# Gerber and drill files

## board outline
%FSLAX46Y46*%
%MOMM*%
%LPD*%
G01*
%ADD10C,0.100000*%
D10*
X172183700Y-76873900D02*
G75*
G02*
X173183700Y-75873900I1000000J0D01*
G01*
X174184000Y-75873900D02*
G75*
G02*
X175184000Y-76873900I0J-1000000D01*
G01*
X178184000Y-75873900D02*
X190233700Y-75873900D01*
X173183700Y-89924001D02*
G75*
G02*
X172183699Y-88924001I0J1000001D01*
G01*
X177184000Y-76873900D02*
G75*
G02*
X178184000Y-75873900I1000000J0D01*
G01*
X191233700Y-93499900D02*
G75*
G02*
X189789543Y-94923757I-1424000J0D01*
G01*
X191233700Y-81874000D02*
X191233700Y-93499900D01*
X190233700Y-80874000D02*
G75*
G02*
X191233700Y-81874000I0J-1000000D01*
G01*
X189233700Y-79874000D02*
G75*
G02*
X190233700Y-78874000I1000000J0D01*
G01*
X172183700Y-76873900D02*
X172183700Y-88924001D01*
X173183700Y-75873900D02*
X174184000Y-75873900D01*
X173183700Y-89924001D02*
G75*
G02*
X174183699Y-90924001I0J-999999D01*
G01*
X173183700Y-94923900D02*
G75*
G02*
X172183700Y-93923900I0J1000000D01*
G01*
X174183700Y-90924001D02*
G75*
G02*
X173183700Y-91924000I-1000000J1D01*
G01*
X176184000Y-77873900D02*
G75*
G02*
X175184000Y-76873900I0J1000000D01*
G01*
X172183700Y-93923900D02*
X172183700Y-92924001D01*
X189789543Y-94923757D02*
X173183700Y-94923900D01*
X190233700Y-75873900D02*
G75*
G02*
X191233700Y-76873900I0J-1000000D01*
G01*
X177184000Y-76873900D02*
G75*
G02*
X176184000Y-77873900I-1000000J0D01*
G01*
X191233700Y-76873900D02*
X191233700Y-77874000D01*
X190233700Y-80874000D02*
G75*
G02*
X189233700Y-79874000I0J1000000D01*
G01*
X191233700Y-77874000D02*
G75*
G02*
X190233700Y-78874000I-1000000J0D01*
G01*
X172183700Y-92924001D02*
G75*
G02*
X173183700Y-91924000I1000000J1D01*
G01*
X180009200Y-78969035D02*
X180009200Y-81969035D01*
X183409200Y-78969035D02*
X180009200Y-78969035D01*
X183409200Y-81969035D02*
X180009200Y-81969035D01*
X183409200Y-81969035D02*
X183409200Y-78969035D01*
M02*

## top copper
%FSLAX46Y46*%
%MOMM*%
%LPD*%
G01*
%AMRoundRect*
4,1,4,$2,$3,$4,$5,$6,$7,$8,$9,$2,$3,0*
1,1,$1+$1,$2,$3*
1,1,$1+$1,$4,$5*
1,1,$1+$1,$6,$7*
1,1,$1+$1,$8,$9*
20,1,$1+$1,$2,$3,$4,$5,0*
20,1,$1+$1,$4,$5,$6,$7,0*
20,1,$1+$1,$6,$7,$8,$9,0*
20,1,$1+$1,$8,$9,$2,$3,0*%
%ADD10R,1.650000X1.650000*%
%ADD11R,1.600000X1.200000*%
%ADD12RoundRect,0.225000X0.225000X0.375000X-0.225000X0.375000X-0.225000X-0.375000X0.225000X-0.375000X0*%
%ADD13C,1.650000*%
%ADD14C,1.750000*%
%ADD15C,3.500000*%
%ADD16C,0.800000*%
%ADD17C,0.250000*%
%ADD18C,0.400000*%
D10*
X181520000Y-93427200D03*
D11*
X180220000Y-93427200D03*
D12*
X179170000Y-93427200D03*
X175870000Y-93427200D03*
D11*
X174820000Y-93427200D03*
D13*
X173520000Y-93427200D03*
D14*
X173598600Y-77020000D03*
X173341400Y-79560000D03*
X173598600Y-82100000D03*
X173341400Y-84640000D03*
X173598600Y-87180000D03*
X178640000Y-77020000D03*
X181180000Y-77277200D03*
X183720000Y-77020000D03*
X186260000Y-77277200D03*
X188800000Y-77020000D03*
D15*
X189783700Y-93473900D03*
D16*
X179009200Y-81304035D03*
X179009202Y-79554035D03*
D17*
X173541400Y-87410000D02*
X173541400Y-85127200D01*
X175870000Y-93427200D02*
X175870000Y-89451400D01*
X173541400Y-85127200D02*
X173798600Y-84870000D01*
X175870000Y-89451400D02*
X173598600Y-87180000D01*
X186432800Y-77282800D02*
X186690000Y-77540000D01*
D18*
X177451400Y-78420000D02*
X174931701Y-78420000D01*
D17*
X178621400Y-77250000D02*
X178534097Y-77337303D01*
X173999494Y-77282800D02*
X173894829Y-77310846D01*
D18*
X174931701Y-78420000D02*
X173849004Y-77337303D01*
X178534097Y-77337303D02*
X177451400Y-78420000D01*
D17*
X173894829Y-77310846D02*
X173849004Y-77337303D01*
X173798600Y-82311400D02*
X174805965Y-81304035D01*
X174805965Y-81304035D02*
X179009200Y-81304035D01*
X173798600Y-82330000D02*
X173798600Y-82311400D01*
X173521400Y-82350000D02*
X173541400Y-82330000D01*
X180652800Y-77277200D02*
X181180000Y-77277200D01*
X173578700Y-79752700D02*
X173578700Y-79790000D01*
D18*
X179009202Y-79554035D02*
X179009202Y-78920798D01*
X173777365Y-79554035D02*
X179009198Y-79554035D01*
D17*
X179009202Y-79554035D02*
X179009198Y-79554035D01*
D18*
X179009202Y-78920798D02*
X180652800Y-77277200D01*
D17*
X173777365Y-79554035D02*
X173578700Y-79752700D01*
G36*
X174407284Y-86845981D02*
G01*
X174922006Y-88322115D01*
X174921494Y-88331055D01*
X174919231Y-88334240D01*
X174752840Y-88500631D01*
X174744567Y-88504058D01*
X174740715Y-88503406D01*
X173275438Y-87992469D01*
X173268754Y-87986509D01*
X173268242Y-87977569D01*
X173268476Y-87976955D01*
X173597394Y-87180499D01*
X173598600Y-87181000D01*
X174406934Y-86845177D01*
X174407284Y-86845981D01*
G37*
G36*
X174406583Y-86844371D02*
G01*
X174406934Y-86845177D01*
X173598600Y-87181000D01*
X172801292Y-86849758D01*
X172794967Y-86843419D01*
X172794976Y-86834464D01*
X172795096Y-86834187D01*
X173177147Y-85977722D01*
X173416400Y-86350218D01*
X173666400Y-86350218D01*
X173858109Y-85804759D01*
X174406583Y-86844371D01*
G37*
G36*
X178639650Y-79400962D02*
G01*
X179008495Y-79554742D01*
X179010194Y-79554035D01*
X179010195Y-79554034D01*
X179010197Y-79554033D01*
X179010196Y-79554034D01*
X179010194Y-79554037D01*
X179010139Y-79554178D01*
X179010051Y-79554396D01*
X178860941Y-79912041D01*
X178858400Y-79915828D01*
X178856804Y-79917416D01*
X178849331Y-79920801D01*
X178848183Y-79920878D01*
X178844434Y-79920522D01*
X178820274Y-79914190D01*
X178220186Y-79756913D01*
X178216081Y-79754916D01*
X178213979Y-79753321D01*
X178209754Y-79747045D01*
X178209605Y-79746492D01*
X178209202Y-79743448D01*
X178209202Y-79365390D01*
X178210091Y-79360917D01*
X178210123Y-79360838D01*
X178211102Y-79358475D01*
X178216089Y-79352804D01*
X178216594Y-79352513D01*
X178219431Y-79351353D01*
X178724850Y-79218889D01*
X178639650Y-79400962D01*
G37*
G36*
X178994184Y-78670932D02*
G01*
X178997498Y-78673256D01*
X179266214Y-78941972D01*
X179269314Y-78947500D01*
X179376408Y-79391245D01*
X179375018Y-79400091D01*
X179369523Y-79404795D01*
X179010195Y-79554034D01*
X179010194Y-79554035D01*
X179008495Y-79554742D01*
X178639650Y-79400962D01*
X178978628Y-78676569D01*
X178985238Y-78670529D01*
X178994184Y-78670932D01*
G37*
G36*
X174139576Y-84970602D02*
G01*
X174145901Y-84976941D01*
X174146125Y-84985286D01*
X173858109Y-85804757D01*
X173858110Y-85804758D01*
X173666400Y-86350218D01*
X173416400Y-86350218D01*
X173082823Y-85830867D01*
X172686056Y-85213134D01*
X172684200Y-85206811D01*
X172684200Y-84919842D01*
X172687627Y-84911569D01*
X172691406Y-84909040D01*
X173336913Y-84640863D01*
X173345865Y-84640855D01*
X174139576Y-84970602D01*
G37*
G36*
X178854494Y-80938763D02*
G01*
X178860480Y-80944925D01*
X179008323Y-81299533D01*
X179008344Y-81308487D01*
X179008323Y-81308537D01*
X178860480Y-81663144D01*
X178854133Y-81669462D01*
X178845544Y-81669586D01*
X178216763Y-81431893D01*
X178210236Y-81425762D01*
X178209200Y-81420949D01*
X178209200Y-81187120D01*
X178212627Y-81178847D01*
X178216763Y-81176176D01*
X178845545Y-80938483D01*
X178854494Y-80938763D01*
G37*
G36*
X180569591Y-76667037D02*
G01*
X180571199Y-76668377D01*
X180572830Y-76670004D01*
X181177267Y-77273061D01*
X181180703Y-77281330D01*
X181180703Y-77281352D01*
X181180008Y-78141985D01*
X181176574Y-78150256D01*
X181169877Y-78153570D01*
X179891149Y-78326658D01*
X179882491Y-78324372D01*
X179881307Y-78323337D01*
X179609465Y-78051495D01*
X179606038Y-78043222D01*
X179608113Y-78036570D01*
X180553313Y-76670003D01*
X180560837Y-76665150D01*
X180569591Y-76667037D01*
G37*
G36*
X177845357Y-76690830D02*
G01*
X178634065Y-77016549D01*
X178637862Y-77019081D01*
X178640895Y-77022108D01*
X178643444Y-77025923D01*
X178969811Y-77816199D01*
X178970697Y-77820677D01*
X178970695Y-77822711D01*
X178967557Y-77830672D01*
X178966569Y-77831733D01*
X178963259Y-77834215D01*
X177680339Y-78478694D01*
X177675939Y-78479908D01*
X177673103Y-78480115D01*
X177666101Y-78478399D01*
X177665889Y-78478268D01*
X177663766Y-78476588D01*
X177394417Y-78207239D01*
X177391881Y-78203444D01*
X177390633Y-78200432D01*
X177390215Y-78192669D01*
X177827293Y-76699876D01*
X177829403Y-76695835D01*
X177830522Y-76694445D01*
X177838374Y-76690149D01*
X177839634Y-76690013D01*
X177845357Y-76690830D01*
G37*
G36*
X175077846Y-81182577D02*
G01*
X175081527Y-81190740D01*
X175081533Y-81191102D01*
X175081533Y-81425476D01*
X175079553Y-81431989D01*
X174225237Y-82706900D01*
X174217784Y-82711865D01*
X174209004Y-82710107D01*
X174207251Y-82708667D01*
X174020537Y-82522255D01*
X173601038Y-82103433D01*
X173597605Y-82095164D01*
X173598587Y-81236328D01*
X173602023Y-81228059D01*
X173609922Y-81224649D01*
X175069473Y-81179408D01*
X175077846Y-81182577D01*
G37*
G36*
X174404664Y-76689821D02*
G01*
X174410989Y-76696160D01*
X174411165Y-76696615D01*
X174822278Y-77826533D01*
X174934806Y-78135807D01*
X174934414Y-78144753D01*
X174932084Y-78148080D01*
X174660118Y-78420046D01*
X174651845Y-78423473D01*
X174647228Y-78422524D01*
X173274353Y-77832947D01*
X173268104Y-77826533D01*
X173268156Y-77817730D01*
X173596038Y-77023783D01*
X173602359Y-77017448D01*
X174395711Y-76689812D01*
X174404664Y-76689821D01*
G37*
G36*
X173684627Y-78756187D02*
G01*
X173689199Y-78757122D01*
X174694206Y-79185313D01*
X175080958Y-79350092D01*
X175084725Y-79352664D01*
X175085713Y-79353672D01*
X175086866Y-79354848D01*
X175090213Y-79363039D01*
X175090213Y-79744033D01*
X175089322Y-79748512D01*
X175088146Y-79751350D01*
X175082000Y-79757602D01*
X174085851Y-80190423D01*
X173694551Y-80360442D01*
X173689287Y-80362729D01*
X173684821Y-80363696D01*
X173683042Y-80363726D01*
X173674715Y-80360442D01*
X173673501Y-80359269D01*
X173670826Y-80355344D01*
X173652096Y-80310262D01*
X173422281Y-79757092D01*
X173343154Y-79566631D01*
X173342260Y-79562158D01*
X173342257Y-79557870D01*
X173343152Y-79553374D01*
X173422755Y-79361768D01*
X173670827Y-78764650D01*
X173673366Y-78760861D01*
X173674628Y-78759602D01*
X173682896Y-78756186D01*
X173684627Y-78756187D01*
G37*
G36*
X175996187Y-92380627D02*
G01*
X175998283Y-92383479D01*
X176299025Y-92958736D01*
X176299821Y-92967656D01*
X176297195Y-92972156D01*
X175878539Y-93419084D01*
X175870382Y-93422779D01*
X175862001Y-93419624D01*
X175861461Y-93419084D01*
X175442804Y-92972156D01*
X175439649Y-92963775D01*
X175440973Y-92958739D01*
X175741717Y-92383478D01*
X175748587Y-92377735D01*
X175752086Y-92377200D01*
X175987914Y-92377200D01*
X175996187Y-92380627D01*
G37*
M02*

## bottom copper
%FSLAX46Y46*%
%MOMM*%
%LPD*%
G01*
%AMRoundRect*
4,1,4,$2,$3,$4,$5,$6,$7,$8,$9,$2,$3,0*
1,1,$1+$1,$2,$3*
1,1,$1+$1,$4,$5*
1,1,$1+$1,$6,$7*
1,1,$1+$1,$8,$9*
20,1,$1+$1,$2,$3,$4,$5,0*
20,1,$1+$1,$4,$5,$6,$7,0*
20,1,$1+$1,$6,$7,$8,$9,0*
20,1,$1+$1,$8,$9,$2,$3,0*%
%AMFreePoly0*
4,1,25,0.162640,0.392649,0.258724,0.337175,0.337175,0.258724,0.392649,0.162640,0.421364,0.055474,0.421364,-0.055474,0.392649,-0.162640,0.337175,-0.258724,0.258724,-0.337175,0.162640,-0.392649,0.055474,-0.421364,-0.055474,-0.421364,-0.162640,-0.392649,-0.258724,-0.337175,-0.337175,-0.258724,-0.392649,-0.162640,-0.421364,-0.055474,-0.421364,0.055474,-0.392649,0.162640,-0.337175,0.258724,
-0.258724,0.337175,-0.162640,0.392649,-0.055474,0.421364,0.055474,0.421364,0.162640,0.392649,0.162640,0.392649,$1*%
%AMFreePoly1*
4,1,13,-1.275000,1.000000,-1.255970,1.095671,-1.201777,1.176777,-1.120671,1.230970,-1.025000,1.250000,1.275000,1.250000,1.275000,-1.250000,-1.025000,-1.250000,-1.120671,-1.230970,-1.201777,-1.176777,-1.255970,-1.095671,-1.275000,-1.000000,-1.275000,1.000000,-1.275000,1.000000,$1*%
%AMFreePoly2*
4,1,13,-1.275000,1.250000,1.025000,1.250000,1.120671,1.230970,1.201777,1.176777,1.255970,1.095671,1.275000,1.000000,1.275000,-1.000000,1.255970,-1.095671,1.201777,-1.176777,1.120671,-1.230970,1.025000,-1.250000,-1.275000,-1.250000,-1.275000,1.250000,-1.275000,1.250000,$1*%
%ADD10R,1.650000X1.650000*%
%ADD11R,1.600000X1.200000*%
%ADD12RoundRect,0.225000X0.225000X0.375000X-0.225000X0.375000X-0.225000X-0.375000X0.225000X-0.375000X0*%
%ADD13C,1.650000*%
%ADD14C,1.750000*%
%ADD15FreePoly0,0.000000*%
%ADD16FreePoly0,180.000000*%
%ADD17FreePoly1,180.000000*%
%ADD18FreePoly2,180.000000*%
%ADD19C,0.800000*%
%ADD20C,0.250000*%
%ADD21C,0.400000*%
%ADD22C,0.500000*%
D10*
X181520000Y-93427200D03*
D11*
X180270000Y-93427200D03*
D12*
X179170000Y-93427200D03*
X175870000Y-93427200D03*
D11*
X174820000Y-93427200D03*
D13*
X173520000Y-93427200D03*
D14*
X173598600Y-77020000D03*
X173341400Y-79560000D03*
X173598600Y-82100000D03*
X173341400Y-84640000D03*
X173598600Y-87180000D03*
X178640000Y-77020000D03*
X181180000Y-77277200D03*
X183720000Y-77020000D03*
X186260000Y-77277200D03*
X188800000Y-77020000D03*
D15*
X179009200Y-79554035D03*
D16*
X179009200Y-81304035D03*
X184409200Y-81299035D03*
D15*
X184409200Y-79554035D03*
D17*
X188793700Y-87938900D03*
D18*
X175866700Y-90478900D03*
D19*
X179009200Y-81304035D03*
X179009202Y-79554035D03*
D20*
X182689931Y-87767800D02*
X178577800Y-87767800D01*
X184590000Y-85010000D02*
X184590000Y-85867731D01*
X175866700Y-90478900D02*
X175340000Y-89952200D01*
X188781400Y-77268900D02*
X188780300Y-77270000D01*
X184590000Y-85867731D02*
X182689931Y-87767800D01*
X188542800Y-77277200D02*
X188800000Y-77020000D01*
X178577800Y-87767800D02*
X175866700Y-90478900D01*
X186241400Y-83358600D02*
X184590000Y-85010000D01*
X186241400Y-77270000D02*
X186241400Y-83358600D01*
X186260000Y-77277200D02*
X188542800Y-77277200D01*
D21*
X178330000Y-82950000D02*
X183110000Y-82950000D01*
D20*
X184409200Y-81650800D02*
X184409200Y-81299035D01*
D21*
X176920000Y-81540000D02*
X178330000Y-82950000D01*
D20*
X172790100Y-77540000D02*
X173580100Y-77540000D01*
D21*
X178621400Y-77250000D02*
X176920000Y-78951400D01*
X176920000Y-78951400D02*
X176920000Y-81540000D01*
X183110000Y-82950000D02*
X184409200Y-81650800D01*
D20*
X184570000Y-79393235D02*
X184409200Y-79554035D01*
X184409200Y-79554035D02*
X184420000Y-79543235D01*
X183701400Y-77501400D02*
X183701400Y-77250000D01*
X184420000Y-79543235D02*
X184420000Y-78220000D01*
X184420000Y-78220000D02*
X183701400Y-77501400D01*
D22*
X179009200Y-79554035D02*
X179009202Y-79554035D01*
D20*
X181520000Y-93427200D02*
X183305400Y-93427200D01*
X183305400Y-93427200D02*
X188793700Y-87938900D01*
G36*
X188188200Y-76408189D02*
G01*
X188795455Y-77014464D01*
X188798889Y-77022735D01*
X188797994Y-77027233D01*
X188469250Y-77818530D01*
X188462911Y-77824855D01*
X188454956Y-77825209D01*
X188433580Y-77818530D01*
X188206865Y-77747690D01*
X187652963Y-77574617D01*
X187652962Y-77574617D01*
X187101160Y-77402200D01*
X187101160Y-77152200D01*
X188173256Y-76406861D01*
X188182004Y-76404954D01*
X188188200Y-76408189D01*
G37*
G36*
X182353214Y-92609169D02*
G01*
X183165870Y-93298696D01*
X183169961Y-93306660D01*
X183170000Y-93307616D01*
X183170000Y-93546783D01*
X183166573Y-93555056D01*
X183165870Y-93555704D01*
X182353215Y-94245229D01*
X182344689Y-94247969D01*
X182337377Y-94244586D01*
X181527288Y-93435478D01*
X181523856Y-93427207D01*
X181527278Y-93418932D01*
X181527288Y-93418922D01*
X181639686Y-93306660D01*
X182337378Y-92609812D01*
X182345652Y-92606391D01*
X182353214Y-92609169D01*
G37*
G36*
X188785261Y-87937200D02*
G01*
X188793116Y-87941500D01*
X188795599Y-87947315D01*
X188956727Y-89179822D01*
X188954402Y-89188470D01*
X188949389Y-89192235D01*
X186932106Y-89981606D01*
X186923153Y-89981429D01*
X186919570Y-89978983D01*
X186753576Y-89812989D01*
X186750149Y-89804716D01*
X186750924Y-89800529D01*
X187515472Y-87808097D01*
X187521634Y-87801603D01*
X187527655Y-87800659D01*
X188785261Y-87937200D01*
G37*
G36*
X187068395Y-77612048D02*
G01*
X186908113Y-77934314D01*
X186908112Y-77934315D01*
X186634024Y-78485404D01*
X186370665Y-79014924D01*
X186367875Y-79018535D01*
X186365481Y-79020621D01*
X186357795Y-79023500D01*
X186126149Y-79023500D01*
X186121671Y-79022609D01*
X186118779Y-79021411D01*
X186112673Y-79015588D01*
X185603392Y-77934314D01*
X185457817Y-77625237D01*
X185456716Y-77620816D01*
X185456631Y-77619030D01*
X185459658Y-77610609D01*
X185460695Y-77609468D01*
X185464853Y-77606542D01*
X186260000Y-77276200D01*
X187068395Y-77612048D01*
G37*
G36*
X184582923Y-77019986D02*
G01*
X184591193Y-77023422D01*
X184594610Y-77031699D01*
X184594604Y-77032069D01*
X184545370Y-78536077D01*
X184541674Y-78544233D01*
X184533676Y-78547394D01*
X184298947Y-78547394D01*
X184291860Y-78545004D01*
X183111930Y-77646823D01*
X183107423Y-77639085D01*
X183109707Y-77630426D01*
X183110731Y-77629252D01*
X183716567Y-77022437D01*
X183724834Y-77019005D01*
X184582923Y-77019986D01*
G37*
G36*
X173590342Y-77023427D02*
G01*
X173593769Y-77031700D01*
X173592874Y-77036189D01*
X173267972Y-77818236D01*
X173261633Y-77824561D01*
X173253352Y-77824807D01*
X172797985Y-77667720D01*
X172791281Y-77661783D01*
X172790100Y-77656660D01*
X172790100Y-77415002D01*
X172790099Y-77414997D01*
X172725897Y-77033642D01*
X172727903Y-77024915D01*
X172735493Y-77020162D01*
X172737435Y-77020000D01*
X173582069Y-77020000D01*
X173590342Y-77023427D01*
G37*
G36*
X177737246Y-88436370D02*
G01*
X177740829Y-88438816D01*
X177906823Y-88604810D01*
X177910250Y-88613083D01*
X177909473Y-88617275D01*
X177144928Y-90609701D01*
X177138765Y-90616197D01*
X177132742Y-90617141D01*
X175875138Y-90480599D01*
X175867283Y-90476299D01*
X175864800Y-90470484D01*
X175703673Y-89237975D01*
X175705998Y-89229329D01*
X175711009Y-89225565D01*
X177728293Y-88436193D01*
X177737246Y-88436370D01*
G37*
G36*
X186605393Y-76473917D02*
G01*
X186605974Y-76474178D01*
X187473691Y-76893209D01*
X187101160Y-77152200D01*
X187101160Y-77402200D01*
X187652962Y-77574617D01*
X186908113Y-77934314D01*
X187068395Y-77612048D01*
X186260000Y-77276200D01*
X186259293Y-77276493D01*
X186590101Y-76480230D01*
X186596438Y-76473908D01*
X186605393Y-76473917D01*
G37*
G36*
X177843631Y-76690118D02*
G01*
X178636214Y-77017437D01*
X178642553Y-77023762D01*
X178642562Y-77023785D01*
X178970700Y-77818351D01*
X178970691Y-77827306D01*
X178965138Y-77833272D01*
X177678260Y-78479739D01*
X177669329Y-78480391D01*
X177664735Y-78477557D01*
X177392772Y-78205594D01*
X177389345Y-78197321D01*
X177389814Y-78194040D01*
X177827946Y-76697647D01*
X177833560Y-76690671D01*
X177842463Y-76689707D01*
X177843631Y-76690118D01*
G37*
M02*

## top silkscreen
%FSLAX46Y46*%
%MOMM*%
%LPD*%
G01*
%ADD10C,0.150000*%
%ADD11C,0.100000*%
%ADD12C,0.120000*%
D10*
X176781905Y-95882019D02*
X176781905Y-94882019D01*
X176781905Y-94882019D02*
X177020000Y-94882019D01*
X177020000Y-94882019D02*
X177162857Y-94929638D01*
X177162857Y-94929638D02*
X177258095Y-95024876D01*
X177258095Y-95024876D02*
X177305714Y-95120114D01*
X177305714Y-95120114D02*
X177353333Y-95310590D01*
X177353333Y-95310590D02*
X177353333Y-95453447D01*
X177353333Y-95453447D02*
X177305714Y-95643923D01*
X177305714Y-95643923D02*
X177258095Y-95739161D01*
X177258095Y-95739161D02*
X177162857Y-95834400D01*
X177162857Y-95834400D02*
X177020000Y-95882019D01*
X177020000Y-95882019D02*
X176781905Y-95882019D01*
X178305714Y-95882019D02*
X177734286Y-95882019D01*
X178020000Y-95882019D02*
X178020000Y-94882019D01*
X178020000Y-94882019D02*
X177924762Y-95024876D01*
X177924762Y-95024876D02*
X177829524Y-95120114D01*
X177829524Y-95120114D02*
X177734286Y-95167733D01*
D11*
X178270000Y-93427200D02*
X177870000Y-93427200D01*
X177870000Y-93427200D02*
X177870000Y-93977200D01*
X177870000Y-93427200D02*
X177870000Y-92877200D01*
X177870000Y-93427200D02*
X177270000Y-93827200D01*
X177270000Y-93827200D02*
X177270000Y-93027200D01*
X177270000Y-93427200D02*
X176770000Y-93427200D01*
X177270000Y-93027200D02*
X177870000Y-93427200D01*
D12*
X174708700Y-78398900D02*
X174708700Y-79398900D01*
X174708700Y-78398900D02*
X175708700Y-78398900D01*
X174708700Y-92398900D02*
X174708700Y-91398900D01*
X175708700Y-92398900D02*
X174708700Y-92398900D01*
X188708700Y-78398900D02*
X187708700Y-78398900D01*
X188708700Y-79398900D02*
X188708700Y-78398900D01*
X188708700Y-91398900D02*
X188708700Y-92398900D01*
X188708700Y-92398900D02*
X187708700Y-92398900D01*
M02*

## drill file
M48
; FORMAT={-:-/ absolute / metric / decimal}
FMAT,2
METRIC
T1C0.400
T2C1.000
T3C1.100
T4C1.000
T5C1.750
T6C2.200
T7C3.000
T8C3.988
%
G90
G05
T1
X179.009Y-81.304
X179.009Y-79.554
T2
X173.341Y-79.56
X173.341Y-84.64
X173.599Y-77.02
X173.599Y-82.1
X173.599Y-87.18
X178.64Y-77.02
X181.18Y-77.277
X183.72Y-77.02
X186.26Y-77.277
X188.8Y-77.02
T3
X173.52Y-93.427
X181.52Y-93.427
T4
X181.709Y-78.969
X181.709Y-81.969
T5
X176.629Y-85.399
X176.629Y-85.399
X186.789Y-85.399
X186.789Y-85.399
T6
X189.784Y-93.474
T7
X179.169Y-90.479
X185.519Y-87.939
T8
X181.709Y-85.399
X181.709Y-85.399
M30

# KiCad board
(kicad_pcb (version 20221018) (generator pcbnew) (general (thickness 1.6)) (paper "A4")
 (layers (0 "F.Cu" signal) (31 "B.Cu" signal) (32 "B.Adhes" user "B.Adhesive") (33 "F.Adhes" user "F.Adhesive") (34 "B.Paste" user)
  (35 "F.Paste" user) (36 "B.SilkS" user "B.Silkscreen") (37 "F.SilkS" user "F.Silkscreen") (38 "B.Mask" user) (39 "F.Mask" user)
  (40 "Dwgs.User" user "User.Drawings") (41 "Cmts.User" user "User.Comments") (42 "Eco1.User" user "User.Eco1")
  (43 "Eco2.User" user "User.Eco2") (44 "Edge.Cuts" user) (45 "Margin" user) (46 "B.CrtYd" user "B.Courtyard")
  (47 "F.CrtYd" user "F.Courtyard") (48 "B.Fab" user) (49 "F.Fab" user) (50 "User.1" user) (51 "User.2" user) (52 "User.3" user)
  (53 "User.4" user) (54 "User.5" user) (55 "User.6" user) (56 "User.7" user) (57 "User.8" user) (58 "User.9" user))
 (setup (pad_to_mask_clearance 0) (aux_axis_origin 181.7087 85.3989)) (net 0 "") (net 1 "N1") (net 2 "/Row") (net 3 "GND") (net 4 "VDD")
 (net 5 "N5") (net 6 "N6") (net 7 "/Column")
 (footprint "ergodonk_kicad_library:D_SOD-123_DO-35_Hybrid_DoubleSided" (layer "F.Cu") (at 177.52 93.4272 180)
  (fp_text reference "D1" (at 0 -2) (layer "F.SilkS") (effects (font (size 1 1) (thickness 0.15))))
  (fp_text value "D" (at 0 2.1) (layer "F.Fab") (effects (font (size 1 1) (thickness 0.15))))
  (fp_line (start -0.75 0) (end -0.35 0) (stroke (width 0.1) (type solid)) (layer "F.SilkS"))
  (fp_line (start -0.35 0) (end -0.35 -0.55) (stroke (width 0.1) (type solid)) (layer "F.SilkS"))
  (fp_line (start -0.35 0) (end -0.35 0.55) (stroke (width 0.1) (type solid)) (layer "F.SilkS"))
  (fp_line (start -0.35 0) (end 0.25 -0.4) (stroke (width 0.1) (type solid)) (layer "F.SilkS"))
  (fp_line (start 0.25 -0.4) (end 0.25 0.4) (stroke (width 0.1) (type solid)) (layer "F.SilkS"))
  (fp_line (start 0.25 0) (end 0.75 0) (stroke (width 0.1) (type solid)) (layer "F.SilkS"))
  (fp_line (start 0.25 0.4) (end -0.35 0) (stroke (width 0.1) (type solid)) (layer "F.SilkS"))
  (pad "1" thru_hole rect (at -4 0 180) (size 1.65 1.65) (drill 1.1) (layers "*.Cu" "*.Mask") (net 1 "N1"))
  (pad "1" smd rect (at -2.75 0 180) (size 1.6 1.2) (layers "B.Cu") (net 1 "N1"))
  (pad "1" smd rect (at -2.7 0 180) (size 1.6 1.2) (layers "F.Cu") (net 1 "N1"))
  (pad "1" smd roundrect (at -1.65 0 180) (size 0.9 1.2) (layers "F.Cu" "F.Paste" "F.Mask") (roundrect_rratio 0.25) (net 1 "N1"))
  (pad "1" smd roundrect (at -1.65 0 180) (size 0.9 1.2) (layers "B.Cu" "B.Paste" "B.Mask") (roundrect_rratio 0.25) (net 1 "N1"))
  (pad "2" smd roundrect (at 1.65 0 180) (size 0.9 1.2) (layers "F.Cu" "F.Paste" "F.Mask") (roundrect_rratio 0.25) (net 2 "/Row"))
  (pad "2" smd roundrect (at 1.65 0 180) (size 0.9 1.2) (layers "B.Cu" "B.Paste" "B.Mask") (roundrect_rratio 0.25) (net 2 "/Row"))
  (pad "2" smd rect (at 2.7 0 180) (size 1.6 1.2) (layers "F.Cu") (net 2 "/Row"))
  (pad "2" smd rect (at 2.7 0 180) (size 1.6 1.2) (layers "B.Cu") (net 2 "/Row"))
  (pad "2" thru_hole circle (at 4 0 180) (size 1.65 1.65) (drill 1.1) (layers "*.Cu" "*.Mask") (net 2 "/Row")))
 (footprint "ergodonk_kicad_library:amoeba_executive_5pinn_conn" (layer "F.Cu") (at 173.47 82.1 -90)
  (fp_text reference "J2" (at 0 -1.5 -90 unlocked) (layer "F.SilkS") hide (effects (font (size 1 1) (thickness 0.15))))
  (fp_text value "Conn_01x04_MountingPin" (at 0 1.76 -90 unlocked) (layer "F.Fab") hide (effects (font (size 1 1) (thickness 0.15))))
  (pad "1" thru_hole circle (at -5.08 -0.1286 90) (size 1.75 1.75) (drill 1) (layers "*.Cu" "*.Mask") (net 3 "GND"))
  (pad "2" thru_hole circle (at -2.54 0.1286 90) (size 1.75 1.75) (drill 1) (layers "*.Cu" "*.Mask") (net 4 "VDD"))
  (pad "3" thru_hole circle (at 0 -0.1286 90) (size 1.75 1.75) (drill 1) (layers "*.Cu" "*.Mask") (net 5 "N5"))
  (pad "4" thru_hole circle (at 2.54 0.1286 90) (size 1.75 1.75) (drill 1) (layers "*.Cu" "*.Mask") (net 2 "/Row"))
  (pad "5" thru_hole circle (at 5.08 -0.1286 90) (size 1.75 1.75) (drill 1) (layers "*.Cu" "*.Mask") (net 2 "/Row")))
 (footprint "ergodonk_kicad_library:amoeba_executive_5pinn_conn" (layer "F.Cu") (at 183.72 77.1486)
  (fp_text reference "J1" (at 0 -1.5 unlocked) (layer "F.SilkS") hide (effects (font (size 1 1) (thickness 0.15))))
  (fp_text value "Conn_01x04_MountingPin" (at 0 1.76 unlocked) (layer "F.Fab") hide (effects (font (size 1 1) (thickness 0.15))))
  (pad "1" thru_hole circle (at -5.08 -0.1286 180) (size 1.75 1.75) (drill 1) (layers "*.Cu" "*.Mask") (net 3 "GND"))
  (pad "2" thru_hole circle (at -2.54 0.1286 180) (size 1.75 1.75) (drill 1) (layers "*.Cu" "*.Mask") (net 4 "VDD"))
  (pad "3" thru_hole circle (at 0 -0.1286 180) (size 1.75 1.75) (drill 1) (layers "*.Cu" "*.Mask") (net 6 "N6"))
  (pad "4" thru_hole circle (at 2.54 0.1286 180) (size 1.75 1.75) (drill 1) (layers "*.Cu" "*.Mask") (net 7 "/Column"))
  (pad "5" thru_hole circle (at 5.08 -0.1286 180) (size 1.75 1.75) (drill 1) (layers "*.Cu" "*.Mask") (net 7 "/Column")))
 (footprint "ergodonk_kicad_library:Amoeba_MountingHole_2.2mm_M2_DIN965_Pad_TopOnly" (layer "F.Cu") (at 189.7837 93.4739)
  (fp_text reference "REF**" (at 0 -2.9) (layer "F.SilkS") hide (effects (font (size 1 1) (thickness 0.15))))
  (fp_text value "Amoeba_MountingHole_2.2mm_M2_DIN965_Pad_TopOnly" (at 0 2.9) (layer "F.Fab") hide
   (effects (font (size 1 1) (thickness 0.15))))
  (pad "" np_thru_hole circle (at 0 0) (size 2.2 2.2) (drill 2.2) (layers "F&B.Cu" "*.Mask"))
  (pad "1" connect circle (at 0 0) (size 3.5 3.5) (layers "F.Cu" "F.Mask")))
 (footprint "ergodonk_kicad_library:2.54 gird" (layer "F.Cu") (at 178.68 86.5)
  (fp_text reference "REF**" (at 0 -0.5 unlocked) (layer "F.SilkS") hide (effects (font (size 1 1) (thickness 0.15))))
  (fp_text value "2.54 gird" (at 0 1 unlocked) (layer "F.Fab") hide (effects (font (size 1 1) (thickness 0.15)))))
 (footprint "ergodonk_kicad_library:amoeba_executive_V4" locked (layer "F.Cu") (at 181.7087 85.3989)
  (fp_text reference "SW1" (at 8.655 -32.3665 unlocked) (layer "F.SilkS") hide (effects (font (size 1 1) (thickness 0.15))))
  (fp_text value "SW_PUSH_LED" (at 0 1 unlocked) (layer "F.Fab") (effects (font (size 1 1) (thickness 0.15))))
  (fp_line (start -7 -7) (end -7 -6) (stroke (width 0.12) (type default)) (layer "F.SilkS"))
  (fp_line (start -7 -7) (end -6 -7) (stroke (width 0.12) (type default)) (layer "F.SilkS"))
  (fp_line (start -7 7) (end -7 6) (stroke (width 0.12) (type default)) (layer "F.SilkS"))
  (fp_line (start -6 7) (end -7 7) (stroke (width 0.12) (type default)) (layer "F.SilkS"))
  (fp_line (start 7 -7) (end 6 -7) (stroke (width 0.12) (type default)) (layer "F.SilkS"))
  (fp_line (start 7 -6) (end 7 -7) (stroke (width 0.12) (type default)) (layer "F.SilkS"))
  (fp_line (start 7 6) (end 7 7) (stroke (width 0.12) (type default)) (layer "F.SilkS"))
  (fp_line (start 7 7) (end 6 7) (stroke (width 0.12) (type default)) (layer "F.SilkS"))
  (fp_line (start -1.6995 -6.429865) (end -1.6995 -3.429865) (stroke (width 0.1) (type solid)) (layer "Edge.Cuts"))
  (fp_line (start 1.7005 -6.429865) (end -1.6995 -6.429865) (stroke (width 0.1) (type solid)) (layer "Edge.Cuts"))
  (fp_line (start 1.7005 -3.429865) (end -1.6995 -3.429865) (stroke (width 0.1) (type solid)) (layer "Edge.Cuts"))
  (fp_line (start 1.7005 -3.429865) (end 1.7005 -6.429865) (stroke (width 0.1) (type solid)) (layer "Edge.Cuts"))
  (pad "" np_thru_hole circle locked (at -5.08 0 180) (size 1.75 1.75) (drill 1.75) (layers "*.Cu" "*.Mask"))
  (pad "" np_thru_hole circle locked (at -5.08 0 180) (size 1.75 1.75) (drill 1.75) (layers "*.Cu" "*.Mask"))
  (pad "" smd roundrect locked (at -2.6895 -5.844813) (size 1.819974 0.850103) (layers "B.Mask") (roundrect_rratio 0.25) (chamfer_ratio 0)
   (chamfer top_right bottom_right) (clearance 0.2) (zone_connect 2))
  (pad "" smd roundrect locked (at -2.689487 -4.094968) (size 1.819974 0.840206) (layers "B.Mask") (roundrect_rratio 0.25) (chamfer_ratio 0)
   (chamfer top_right bottom_right) (clearance 0.2) (zone_connect 2))
  (pad "" np_thru_hole circle locked (at -2.54 5.08 180) (size 3 3) (drill 3) (layers "*.Cu" "*.Mask"))
  (pad "" np_thru_hole circle locked (at 0 0 180) (size 3.9878 3.9878) (drill 3.9878) (layers "*.Cu" "*.Mask"))
  (pad "" np_thru_hole circle locked (at 0 0 180) (size 3.9878 3.9878) (drill 3.9878) (layers "*.Cu" "*.Mask"))
  (pad "" np_thru_hole circle locked (at 0.0005 -6.429865 180) (size 1 1) (drill 1) (layers "F&B.Cu" "*.Mask"))
  (pad "" np_thru_hole circle locked (at 0.0005 -3.430135 180) (size 1 1) (drill 1) (layers "F&B.Cu" "*.Mask"))
  (pad "" smd rect locked (at 2.470506 -4.089865 180) (size 1.379987 0.840206) (layers "B.Mask") (clearance 0.2) (zone_connect 2))
  (pad "" smd roundrect locked (at 2.6905 -5.839865 180) (size 1.819974 0.840206) (layers "B.Mask") (roundrect_rratio 0.25)
   (chamfer_ratio 0) (chamfer top_right bottom_right) (clearance 0.2) (zone_connect 2))
  (pad "" smd roundrect locked (at 2.855493 -4.089865 180) (size 1.489986 0.840206) (layers "B.Mask") (roundrect_rratio 0.25)
   (chamfer_ratio 0.5) (chamfer top_left) (clearance 0.2) (zone_connect 2))
  (pad "" np_thru_hole circle locked (at 3.81 2.54 180) (size 3 3) (drill 3) (layers "*.Cu" "*.Mask"))
  (pad "" np_thru_hole circle locked (at 5.08 0 180) (size 1.75 1.75) (drill 1.75) (layers "*.Cu" "*.Mask"))
  (pad "" np_thru_hole circle locked (at 5.08 0 180) (size 1.75 1.75) (drill 1.75) (layers "*.Cu" "*.Mask"))
  (pad "1" smd custom locked (at -2.6995 -5.844865) (size 0.85 0.85) (layers "B.Cu") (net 4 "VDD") (clearance 0.2) (zone_connect 2)
   (thermal_bridge_angle 45) (options (clearance outline) (anchor circle)) (primitives))
  (pad "2" smd custom locked (at -2.6995 -4.094865 180) (size 0.85 0.85) (layers "B.Cu") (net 5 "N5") (clearance 0.2) (zone_connect 2)
   (thermal_bridge_angle 45) (options (clearance outline) (anchor circle)) (primitives))
  (pad "3" smd custom locked (at 2.7005 -4.099865 180) (size 0.85 0.85) (layers "B.Cu") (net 3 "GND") (clearance 0.2) (zone_connect 2)
   (thermal_bridge_angle 45) (options (clearance outline) (anchor circle)) (primitives))
  (pad "4" smd custom locked (at 2.7005 -5.844865) (size 0.85 0.85) (layers "B.Cu") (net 6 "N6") (clearance 0.2) (zone_connect 2)
   (thermal_bridge_angle 45) (options (clearance outline) (anchor circle)) (primitives))
  (pad "5" smd roundrect locked (at 7.085 2.54 180) (size 2.55 2.5) (layers "B.Cu" "B.Paste" "B.Mask") (roundrect_rratio 0.1)
   (chamfer_ratio 0) (chamfer top_right bottom_right) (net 1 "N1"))
  (pad "6" smd roundrect locked (at -5.842 5.08 180) (size 2.55 2.5) (layers "B.Cu" "B.Paste" "B.Mask") (roundrect_rratio 0.1)
   (chamfer_ratio 0) (chamfer top_left bottom_left) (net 7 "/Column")))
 (gr_arc (start 172.1837 76.8739) (mid 172.476594 76.166795) (end 173.1837 75.8739) (stroke (width 0.1) (type default)) (layer "Edge.Cuts"))
 (gr_arc (start 174.184 75.8739) (mid 174.891107 76.166793) (end 175.184 76.8739) (stroke (width 0.1) (type default)) (layer "Edge.Cuts"))
 (gr_line (start 178.184 75.8739) (end 190.2337 75.8739) (stroke (width 0.1) (type default)) (layer "Edge.Cuts"))
 (gr_arc (start 173.1837 89.924001) (mid 172.476593 89.631108) (end 172.1837 88.924001) (stroke (width 0.1) (type default))
  (layer "Edge.Cuts"))
 (gr_arc (start 177.184 76.8739) (mid 177.476893 76.166793) (end 178.184 75.8739) (stroke (width 0.1) (type default)) (layer "Edge.Cuts"))
 (gr_arc (start 191.2337 93.4999) (mid 190.809468 94.513922) (end 189.789543 94.923757) (stroke (width 0.1) (type default))
  (layer "Edge.Cuts"))
 (gr_line (start 191.2337 81.874) (end 191.2337 93.4999) (stroke (width 0.1) (type default)) (layer "Edge.Cuts"))
 (gr_arc (start 190.2337 80.874) (mid 190.940807 81.166893) (end 191.2337 81.874) (stroke (width 0.1) (type default)) (layer "Edge.Cuts"))
 (gr_arc (start 189.2337 79.874) (mid 189.526593 79.166893) (end 190.2337 78.874) (stroke (width 0.1) (type default)) (layer "Edge.Cuts"))
 (gr_line (start 172.1837 76.8739) (end 172.1837 88.924001) (stroke (width 0.1) (type default)) (layer "Edge.Cuts"))
 (gr_line (start 173.1837 75.8739) (end 174.184 75.8739) (stroke (width 0.1) (type default)) (layer "Edge.Cuts"))
 (gr_arc (start 173.1837 89.924001) (mid 173.890807 90.216894) (end 174.1837 90.924001) (stroke (width 0.1) (type default))
  (layer "Edge.Cuts"))
 (gr_arc (start 173.1837 94.9239) (mid 172.476593 94.631007) (end 172.1837 93.9239) (stroke (width 0.1) (type default)) (layer "Edge.Cuts"))
 (gr_arc (start 174.1837 90.924001) (mid 173.890807 91.631108) (end 173.1837 91.924001) (stroke (width 0.1) (type default))
  (layer "Edge.Cuts"))
 (gr_arc (start 176.184 77.8739) (mid 175.476893 77.581007) (end 175.184 76.8739) (stroke (width 0.1) (type default)) (layer "Edge.Cuts"))
 (gr_line (start 172.1837 93.9239) (end 172.1837 92.924001) (stroke (width 0.1) (type default)) (layer "Edge.Cuts"))
 (gr_line (start 189.789543 94.923757) (end 173.1837 94.9239) (stroke (width 0.1) (type default)) (layer "Edge.Cuts"))
 (gr_arc (start 190.2337 75.8739) (mid 190.940805 76.166795) (end 191.2337 76.8739) (stroke (width 0.1) (type default)) (layer "Edge.Cuts"))
 (gr_arc (start 177.184 76.8739) (mid 176.891107 77.581007) (end 176.184 77.8739) (stroke (width 0.1) (type default)) (layer "Edge.Cuts"))
 (gr_line (start 191.2337 76.8739) (end 191.2337 77.874) (stroke (width 0.1) (type default)) (layer "Edge.Cuts"))
 (gr_arc (start 190.2337 80.874) (mid 189.526593 80.581107) (end 189.2337 79.874) (stroke (width 0.1) (type default)) (layer "Edge.Cuts"))
 (gr_arc (start 191.2337 77.874) (mid 190.940807 78.581107) (end 190.2337 78.874) (stroke (width 0.1) (type default)) (layer "Edge.Cuts"))
 (gr_arc (start 172.1837 92.924001) (mid 172.476593 92.216894) (end 173.1837 91.924001) (stroke (width 0.1) (type default))
  (layer "Edge.Cuts"))
 (segment (start 173.5414 87.41) (end 173.5414 85.1272) (width 0.25) (layer "F.Cu") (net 2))
 (segment (start 175.87 93.4272) (end 175.87 89.4514) (width 0.25) (layer "F.Cu") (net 2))
 (segment (start 173.5414 85.1272) (end 173.7986 84.87) (width 0.25) (layer "F.Cu") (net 2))
 (segment (start 175.87 89.4514) (end 173.5986 87.18) (width 0.25) (layer "F.Cu") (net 2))
 (segment (start 186.4328 77.2828) (end 186.69 77.54) (width 0.25) (layer "F.Cu") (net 7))
 (segment (start 182.689931 87.7678) (end 178.5778 87.7678) (width 0.25) (layer "B.Cu") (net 7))
 (segment (start 184.59 85.01) (end 184.59 85.867731) (width 0.25) (layer "B.Cu") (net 7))
 (segment (start 175.8667 90.4789) (end 175.34 89.9522) (width 0.25) (layer "B.Cu") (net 7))
 (segment (start 188.7814 77.2689) (end 188.7803 77.27) (width 0.25) (layer "B.Cu") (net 7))
 (segment (start 184.59 85.867731) (end 182.689931 87.7678) (width 0.25) (layer "B.Cu") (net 7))
 (segment (start 188.5428 77.2772) (end 188.8 77.02) (width 0.25) (layer "B.Cu") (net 7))
 (segment (start 178.5778 87.7678) (end 175.8667 90.4789) (width 0.25) (layer "B.Cu") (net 7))
 (segment (start 186.2414 83.3586) (end 184.59 85.01) (width 0.25) (layer "B.Cu") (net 7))
 (segment (start 186.2414 77.27) (end 186.2414 83.3586) (width 0.25) (layer "B.Cu") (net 7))
 (segment (start 186.26 77.2772) (end 188.5428 77.2772) (width 0.25) (layer "B.Cu") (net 7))
 (segment (start 177.4514 78.42) (end 174.931701 78.42) (width 0.4) (layer "F.Cu") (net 3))
 (segment (start 178.6214 77.25) (end 178.534097 77.337303) (width 0.25) (layer "F.Cu") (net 3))
 (segment (start 173.999494 77.2828) (end 173.894829 77.310846) (width 0.25) (layer "F.Cu") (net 3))
 (segment (start 174.931701 78.42) (end 173.849004 77.337303) (width 0.4) (layer "F.Cu") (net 3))
 (segment (start 178.534097 77.337303) (end 177.4514 78.42) (width 0.4) (layer "F.Cu") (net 3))
 (segment (start 173.894829 77.310846) (end 173.849004 77.337303) (width 0.25) (layer "F.Cu") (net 3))
 (segment (start 178.33 82.95) (end 183.11 82.95) (width 0.4) (layer "B.Cu") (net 3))
 (segment (start 184.4092 81.6508) (end 184.4092 81.299035) (width 0.25) (layer "B.Cu") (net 3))
 (segment (start 176.92 81.54) (end 178.33 82.95) (width 0.4) (layer "B.Cu") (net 3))
 (segment (start 172.7901 77.54) (end 173.5801 77.54) (width 0.25) (layer "B.Cu") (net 3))
 (segment (start 178.6214 77.25) (end 176.92 78.9514) (width 0.4) (layer "B.Cu") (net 3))
 (segment (start 176.92 78.9514) (end 176.92 81.54) (width 0.4) (layer "B.Cu") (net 3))
 (segment (start 183.11 82.95) (end 184.4092 81.6508) (width 0.4) (layer "B.Cu") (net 3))
 (segment (start 184.57 79.393235) (end 184.4092 79.554035) (width 0.25) (layer "B.Cu") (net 6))
 (segment (start 184.4092 79.554035) (end 184.42 79.543235) (width 0.25) (layer "B.Cu") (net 6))
 (segment (start 183.7014 77.5014) (end 183.7014 77.25) (width 0.25) (layer "B.Cu") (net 6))
 (segment (start 184.42 79.543235) (end 184.42 78.22) (width 0.25) (layer "B.Cu") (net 6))
 (segment (start 184.42 78.22) (end 183.7014 77.5014) (width 0.25) (layer "B.Cu") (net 6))
 (segment (start 173.7986 82.3114) (end 174.805965 81.304035) (width 0.25) (layer "F.Cu") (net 5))
 (segment (start 174.805965 81.304035) (end 179.0092 81.304035) (width 0.25) (layer "F.Cu") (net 5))
 (segment (start 173.7986 82.33) (end 173.7986 82.3114) (width 0.25) (layer "F.Cu") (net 5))
 (segment (start 173.5214 82.35) (end 173.5414 82.33) (width 0.25) (layer "F.Cu") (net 5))
 (via (at 179.0092 81.304035) (size 0.8) (drill 0.4) (layers "F.Cu" "B.Cu") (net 5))
 (segment (start 180.6528 77.2772) (end 181.18 77.2772) (width 0.25) (layer "F.Cu") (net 4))
 (segment (start 173.5787 79.7527) (end 173.5787 79.79) (width 0.25) (layer "F.Cu") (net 4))
 (segment (start 179.009202 79.554035) (end 179.009202 78.920798) (width 0.4) (layer "F.Cu") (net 4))
 (segment (start 173.777365 79.554035) (end 179.009198 79.554035) (width 0.4) (layer "F.Cu") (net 4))
 (segment (start 179.009202 79.554035) (end 179.009198 79.554035) (width 0.25) (layer "F.Cu") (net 4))
 (segment (start 179.009202 78.920798) (end 180.6528 77.2772) (width 0.4) (layer "F.Cu") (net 4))
 (segment (start 173.777365 79.554035) (end 173.5787 79.7527) (width 0.25) (layer "F.Cu") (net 4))
 (via (at 179.009202 79.554035) (size 0.8) (drill 0.4) (layers "F.Cu" "B.Cu") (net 4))
 (segment (start 179.0092 79.554035) (end 179.009202 79.554035) (width 0.5) (layer "B.Cu") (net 4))
 (segment (start 181.52 93.4272) (end 183.3054 93.4272) (width 0.25) (layer "B.Cu") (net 1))
 (segment (start 183.3054 93.4272) (end 188.7937 87.9389) (width 0.25) (layer "B.Cu") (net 1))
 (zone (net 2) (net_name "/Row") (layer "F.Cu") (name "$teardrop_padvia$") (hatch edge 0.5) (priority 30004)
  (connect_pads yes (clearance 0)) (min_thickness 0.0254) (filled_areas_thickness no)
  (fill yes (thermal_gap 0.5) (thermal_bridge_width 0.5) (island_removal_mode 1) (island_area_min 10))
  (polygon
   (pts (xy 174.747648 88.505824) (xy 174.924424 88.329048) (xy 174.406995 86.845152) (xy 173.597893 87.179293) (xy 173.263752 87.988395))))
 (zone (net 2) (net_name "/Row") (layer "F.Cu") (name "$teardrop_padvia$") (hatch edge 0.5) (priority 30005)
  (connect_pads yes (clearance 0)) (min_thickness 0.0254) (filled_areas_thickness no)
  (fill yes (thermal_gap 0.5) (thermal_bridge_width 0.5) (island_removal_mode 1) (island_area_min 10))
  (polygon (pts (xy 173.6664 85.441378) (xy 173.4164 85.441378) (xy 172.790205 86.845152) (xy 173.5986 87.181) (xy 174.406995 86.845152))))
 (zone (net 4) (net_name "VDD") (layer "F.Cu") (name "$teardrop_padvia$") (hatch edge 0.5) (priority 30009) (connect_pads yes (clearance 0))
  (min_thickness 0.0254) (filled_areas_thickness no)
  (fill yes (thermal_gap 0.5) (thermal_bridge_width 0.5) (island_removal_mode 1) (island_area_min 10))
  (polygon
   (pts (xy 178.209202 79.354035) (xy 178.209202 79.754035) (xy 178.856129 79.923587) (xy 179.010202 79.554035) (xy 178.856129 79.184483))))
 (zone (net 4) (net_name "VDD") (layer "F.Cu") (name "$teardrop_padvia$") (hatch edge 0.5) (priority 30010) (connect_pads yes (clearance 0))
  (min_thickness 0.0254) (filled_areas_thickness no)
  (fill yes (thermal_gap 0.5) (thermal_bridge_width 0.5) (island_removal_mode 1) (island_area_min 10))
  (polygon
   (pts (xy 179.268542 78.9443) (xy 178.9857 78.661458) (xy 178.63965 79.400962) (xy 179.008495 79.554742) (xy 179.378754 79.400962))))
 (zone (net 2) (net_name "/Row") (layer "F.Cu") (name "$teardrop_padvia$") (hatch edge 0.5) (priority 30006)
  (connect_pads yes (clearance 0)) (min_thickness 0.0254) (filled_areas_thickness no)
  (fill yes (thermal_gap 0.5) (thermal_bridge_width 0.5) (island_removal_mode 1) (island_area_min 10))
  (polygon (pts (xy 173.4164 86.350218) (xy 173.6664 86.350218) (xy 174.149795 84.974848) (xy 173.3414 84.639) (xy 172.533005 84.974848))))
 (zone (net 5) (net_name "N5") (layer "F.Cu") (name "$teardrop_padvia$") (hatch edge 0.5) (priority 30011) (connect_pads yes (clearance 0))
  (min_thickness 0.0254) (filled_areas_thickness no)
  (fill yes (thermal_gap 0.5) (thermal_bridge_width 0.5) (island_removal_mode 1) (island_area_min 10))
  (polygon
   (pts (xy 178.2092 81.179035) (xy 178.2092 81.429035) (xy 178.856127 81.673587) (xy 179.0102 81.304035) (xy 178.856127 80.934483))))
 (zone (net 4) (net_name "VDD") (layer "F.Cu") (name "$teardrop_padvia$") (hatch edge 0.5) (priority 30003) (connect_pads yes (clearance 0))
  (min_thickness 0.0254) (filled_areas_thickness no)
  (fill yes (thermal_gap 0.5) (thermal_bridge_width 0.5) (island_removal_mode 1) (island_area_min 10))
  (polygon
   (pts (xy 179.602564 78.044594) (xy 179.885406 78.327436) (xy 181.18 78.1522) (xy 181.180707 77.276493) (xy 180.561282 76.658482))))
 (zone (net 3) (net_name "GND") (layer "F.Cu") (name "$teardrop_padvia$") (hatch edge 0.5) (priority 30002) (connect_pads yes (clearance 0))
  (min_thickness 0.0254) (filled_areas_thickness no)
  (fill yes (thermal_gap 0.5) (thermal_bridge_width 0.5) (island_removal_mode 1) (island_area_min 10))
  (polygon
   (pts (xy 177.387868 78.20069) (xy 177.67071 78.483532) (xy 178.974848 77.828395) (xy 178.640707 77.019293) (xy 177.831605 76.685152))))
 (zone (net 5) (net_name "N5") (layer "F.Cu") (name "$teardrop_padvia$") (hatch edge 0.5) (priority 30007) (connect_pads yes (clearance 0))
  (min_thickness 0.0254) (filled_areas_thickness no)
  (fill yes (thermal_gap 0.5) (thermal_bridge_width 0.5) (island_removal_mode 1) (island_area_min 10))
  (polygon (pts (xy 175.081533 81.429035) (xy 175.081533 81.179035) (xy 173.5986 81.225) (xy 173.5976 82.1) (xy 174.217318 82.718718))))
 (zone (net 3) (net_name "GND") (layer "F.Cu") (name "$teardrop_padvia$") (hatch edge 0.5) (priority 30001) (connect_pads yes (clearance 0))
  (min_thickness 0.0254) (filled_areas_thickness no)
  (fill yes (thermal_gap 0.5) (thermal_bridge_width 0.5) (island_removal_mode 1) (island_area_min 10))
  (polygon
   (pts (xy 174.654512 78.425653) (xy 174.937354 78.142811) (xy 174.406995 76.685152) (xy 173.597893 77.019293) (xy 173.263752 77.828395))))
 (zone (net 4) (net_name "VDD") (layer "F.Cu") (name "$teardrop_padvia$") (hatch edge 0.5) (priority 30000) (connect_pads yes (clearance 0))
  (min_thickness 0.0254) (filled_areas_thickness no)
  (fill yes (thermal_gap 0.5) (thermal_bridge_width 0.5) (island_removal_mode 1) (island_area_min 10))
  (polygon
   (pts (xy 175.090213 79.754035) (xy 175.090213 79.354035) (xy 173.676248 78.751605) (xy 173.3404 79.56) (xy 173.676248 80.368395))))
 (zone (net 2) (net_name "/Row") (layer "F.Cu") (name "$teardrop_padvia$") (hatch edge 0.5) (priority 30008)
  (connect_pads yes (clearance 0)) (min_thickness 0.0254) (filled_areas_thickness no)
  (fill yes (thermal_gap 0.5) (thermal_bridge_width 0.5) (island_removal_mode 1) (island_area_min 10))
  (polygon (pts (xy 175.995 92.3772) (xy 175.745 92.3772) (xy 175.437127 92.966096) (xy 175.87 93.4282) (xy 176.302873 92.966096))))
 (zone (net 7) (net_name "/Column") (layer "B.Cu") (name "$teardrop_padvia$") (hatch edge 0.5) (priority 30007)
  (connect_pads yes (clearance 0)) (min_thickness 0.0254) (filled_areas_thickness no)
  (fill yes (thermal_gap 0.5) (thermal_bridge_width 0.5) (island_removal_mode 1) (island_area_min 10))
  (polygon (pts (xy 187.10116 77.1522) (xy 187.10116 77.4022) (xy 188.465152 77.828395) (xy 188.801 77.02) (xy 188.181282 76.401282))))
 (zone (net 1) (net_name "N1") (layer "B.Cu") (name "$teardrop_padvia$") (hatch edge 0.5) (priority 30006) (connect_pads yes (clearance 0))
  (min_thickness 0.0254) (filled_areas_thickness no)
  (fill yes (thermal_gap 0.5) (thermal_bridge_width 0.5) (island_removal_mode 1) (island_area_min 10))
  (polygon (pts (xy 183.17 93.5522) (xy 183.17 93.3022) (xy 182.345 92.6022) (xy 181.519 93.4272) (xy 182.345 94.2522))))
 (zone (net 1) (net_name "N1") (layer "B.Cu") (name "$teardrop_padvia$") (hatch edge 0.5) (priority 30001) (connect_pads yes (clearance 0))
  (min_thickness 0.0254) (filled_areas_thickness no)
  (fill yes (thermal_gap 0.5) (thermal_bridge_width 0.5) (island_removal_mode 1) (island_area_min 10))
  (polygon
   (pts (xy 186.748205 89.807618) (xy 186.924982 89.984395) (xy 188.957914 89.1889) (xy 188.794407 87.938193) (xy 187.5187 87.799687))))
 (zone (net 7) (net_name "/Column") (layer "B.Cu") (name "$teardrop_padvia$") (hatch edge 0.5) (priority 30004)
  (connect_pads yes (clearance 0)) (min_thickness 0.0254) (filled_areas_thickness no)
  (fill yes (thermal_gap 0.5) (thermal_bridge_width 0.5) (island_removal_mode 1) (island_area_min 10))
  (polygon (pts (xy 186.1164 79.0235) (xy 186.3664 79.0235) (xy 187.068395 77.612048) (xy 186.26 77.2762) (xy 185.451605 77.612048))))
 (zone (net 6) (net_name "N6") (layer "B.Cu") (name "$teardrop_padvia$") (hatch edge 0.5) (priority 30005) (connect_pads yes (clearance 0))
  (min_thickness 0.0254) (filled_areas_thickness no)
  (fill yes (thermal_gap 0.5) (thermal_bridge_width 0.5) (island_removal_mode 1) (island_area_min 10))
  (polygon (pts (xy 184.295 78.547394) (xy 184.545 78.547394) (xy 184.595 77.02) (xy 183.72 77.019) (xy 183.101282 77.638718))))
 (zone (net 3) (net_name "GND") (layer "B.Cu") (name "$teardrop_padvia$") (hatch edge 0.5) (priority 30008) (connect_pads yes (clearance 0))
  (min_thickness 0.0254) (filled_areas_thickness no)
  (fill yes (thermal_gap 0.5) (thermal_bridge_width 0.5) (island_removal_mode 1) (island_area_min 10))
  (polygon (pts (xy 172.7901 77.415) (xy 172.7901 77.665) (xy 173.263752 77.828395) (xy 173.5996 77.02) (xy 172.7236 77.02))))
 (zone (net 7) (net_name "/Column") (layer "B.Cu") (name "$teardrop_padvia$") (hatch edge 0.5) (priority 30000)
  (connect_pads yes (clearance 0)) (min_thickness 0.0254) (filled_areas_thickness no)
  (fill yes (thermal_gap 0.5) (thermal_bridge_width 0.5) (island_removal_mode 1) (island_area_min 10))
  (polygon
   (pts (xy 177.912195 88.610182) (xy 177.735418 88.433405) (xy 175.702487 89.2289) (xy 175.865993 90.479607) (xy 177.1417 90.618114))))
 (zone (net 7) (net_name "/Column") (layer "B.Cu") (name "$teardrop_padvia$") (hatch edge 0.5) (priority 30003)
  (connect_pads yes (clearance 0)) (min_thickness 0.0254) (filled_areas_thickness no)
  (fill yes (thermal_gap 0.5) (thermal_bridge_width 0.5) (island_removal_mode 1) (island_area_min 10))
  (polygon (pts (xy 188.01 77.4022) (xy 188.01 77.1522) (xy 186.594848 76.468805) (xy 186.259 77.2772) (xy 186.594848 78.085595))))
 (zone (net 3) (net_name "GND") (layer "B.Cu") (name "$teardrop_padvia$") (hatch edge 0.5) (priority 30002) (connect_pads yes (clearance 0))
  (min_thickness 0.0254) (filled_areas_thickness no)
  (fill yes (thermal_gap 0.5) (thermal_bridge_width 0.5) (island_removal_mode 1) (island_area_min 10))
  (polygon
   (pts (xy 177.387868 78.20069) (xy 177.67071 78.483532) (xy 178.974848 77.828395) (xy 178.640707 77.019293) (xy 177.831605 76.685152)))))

